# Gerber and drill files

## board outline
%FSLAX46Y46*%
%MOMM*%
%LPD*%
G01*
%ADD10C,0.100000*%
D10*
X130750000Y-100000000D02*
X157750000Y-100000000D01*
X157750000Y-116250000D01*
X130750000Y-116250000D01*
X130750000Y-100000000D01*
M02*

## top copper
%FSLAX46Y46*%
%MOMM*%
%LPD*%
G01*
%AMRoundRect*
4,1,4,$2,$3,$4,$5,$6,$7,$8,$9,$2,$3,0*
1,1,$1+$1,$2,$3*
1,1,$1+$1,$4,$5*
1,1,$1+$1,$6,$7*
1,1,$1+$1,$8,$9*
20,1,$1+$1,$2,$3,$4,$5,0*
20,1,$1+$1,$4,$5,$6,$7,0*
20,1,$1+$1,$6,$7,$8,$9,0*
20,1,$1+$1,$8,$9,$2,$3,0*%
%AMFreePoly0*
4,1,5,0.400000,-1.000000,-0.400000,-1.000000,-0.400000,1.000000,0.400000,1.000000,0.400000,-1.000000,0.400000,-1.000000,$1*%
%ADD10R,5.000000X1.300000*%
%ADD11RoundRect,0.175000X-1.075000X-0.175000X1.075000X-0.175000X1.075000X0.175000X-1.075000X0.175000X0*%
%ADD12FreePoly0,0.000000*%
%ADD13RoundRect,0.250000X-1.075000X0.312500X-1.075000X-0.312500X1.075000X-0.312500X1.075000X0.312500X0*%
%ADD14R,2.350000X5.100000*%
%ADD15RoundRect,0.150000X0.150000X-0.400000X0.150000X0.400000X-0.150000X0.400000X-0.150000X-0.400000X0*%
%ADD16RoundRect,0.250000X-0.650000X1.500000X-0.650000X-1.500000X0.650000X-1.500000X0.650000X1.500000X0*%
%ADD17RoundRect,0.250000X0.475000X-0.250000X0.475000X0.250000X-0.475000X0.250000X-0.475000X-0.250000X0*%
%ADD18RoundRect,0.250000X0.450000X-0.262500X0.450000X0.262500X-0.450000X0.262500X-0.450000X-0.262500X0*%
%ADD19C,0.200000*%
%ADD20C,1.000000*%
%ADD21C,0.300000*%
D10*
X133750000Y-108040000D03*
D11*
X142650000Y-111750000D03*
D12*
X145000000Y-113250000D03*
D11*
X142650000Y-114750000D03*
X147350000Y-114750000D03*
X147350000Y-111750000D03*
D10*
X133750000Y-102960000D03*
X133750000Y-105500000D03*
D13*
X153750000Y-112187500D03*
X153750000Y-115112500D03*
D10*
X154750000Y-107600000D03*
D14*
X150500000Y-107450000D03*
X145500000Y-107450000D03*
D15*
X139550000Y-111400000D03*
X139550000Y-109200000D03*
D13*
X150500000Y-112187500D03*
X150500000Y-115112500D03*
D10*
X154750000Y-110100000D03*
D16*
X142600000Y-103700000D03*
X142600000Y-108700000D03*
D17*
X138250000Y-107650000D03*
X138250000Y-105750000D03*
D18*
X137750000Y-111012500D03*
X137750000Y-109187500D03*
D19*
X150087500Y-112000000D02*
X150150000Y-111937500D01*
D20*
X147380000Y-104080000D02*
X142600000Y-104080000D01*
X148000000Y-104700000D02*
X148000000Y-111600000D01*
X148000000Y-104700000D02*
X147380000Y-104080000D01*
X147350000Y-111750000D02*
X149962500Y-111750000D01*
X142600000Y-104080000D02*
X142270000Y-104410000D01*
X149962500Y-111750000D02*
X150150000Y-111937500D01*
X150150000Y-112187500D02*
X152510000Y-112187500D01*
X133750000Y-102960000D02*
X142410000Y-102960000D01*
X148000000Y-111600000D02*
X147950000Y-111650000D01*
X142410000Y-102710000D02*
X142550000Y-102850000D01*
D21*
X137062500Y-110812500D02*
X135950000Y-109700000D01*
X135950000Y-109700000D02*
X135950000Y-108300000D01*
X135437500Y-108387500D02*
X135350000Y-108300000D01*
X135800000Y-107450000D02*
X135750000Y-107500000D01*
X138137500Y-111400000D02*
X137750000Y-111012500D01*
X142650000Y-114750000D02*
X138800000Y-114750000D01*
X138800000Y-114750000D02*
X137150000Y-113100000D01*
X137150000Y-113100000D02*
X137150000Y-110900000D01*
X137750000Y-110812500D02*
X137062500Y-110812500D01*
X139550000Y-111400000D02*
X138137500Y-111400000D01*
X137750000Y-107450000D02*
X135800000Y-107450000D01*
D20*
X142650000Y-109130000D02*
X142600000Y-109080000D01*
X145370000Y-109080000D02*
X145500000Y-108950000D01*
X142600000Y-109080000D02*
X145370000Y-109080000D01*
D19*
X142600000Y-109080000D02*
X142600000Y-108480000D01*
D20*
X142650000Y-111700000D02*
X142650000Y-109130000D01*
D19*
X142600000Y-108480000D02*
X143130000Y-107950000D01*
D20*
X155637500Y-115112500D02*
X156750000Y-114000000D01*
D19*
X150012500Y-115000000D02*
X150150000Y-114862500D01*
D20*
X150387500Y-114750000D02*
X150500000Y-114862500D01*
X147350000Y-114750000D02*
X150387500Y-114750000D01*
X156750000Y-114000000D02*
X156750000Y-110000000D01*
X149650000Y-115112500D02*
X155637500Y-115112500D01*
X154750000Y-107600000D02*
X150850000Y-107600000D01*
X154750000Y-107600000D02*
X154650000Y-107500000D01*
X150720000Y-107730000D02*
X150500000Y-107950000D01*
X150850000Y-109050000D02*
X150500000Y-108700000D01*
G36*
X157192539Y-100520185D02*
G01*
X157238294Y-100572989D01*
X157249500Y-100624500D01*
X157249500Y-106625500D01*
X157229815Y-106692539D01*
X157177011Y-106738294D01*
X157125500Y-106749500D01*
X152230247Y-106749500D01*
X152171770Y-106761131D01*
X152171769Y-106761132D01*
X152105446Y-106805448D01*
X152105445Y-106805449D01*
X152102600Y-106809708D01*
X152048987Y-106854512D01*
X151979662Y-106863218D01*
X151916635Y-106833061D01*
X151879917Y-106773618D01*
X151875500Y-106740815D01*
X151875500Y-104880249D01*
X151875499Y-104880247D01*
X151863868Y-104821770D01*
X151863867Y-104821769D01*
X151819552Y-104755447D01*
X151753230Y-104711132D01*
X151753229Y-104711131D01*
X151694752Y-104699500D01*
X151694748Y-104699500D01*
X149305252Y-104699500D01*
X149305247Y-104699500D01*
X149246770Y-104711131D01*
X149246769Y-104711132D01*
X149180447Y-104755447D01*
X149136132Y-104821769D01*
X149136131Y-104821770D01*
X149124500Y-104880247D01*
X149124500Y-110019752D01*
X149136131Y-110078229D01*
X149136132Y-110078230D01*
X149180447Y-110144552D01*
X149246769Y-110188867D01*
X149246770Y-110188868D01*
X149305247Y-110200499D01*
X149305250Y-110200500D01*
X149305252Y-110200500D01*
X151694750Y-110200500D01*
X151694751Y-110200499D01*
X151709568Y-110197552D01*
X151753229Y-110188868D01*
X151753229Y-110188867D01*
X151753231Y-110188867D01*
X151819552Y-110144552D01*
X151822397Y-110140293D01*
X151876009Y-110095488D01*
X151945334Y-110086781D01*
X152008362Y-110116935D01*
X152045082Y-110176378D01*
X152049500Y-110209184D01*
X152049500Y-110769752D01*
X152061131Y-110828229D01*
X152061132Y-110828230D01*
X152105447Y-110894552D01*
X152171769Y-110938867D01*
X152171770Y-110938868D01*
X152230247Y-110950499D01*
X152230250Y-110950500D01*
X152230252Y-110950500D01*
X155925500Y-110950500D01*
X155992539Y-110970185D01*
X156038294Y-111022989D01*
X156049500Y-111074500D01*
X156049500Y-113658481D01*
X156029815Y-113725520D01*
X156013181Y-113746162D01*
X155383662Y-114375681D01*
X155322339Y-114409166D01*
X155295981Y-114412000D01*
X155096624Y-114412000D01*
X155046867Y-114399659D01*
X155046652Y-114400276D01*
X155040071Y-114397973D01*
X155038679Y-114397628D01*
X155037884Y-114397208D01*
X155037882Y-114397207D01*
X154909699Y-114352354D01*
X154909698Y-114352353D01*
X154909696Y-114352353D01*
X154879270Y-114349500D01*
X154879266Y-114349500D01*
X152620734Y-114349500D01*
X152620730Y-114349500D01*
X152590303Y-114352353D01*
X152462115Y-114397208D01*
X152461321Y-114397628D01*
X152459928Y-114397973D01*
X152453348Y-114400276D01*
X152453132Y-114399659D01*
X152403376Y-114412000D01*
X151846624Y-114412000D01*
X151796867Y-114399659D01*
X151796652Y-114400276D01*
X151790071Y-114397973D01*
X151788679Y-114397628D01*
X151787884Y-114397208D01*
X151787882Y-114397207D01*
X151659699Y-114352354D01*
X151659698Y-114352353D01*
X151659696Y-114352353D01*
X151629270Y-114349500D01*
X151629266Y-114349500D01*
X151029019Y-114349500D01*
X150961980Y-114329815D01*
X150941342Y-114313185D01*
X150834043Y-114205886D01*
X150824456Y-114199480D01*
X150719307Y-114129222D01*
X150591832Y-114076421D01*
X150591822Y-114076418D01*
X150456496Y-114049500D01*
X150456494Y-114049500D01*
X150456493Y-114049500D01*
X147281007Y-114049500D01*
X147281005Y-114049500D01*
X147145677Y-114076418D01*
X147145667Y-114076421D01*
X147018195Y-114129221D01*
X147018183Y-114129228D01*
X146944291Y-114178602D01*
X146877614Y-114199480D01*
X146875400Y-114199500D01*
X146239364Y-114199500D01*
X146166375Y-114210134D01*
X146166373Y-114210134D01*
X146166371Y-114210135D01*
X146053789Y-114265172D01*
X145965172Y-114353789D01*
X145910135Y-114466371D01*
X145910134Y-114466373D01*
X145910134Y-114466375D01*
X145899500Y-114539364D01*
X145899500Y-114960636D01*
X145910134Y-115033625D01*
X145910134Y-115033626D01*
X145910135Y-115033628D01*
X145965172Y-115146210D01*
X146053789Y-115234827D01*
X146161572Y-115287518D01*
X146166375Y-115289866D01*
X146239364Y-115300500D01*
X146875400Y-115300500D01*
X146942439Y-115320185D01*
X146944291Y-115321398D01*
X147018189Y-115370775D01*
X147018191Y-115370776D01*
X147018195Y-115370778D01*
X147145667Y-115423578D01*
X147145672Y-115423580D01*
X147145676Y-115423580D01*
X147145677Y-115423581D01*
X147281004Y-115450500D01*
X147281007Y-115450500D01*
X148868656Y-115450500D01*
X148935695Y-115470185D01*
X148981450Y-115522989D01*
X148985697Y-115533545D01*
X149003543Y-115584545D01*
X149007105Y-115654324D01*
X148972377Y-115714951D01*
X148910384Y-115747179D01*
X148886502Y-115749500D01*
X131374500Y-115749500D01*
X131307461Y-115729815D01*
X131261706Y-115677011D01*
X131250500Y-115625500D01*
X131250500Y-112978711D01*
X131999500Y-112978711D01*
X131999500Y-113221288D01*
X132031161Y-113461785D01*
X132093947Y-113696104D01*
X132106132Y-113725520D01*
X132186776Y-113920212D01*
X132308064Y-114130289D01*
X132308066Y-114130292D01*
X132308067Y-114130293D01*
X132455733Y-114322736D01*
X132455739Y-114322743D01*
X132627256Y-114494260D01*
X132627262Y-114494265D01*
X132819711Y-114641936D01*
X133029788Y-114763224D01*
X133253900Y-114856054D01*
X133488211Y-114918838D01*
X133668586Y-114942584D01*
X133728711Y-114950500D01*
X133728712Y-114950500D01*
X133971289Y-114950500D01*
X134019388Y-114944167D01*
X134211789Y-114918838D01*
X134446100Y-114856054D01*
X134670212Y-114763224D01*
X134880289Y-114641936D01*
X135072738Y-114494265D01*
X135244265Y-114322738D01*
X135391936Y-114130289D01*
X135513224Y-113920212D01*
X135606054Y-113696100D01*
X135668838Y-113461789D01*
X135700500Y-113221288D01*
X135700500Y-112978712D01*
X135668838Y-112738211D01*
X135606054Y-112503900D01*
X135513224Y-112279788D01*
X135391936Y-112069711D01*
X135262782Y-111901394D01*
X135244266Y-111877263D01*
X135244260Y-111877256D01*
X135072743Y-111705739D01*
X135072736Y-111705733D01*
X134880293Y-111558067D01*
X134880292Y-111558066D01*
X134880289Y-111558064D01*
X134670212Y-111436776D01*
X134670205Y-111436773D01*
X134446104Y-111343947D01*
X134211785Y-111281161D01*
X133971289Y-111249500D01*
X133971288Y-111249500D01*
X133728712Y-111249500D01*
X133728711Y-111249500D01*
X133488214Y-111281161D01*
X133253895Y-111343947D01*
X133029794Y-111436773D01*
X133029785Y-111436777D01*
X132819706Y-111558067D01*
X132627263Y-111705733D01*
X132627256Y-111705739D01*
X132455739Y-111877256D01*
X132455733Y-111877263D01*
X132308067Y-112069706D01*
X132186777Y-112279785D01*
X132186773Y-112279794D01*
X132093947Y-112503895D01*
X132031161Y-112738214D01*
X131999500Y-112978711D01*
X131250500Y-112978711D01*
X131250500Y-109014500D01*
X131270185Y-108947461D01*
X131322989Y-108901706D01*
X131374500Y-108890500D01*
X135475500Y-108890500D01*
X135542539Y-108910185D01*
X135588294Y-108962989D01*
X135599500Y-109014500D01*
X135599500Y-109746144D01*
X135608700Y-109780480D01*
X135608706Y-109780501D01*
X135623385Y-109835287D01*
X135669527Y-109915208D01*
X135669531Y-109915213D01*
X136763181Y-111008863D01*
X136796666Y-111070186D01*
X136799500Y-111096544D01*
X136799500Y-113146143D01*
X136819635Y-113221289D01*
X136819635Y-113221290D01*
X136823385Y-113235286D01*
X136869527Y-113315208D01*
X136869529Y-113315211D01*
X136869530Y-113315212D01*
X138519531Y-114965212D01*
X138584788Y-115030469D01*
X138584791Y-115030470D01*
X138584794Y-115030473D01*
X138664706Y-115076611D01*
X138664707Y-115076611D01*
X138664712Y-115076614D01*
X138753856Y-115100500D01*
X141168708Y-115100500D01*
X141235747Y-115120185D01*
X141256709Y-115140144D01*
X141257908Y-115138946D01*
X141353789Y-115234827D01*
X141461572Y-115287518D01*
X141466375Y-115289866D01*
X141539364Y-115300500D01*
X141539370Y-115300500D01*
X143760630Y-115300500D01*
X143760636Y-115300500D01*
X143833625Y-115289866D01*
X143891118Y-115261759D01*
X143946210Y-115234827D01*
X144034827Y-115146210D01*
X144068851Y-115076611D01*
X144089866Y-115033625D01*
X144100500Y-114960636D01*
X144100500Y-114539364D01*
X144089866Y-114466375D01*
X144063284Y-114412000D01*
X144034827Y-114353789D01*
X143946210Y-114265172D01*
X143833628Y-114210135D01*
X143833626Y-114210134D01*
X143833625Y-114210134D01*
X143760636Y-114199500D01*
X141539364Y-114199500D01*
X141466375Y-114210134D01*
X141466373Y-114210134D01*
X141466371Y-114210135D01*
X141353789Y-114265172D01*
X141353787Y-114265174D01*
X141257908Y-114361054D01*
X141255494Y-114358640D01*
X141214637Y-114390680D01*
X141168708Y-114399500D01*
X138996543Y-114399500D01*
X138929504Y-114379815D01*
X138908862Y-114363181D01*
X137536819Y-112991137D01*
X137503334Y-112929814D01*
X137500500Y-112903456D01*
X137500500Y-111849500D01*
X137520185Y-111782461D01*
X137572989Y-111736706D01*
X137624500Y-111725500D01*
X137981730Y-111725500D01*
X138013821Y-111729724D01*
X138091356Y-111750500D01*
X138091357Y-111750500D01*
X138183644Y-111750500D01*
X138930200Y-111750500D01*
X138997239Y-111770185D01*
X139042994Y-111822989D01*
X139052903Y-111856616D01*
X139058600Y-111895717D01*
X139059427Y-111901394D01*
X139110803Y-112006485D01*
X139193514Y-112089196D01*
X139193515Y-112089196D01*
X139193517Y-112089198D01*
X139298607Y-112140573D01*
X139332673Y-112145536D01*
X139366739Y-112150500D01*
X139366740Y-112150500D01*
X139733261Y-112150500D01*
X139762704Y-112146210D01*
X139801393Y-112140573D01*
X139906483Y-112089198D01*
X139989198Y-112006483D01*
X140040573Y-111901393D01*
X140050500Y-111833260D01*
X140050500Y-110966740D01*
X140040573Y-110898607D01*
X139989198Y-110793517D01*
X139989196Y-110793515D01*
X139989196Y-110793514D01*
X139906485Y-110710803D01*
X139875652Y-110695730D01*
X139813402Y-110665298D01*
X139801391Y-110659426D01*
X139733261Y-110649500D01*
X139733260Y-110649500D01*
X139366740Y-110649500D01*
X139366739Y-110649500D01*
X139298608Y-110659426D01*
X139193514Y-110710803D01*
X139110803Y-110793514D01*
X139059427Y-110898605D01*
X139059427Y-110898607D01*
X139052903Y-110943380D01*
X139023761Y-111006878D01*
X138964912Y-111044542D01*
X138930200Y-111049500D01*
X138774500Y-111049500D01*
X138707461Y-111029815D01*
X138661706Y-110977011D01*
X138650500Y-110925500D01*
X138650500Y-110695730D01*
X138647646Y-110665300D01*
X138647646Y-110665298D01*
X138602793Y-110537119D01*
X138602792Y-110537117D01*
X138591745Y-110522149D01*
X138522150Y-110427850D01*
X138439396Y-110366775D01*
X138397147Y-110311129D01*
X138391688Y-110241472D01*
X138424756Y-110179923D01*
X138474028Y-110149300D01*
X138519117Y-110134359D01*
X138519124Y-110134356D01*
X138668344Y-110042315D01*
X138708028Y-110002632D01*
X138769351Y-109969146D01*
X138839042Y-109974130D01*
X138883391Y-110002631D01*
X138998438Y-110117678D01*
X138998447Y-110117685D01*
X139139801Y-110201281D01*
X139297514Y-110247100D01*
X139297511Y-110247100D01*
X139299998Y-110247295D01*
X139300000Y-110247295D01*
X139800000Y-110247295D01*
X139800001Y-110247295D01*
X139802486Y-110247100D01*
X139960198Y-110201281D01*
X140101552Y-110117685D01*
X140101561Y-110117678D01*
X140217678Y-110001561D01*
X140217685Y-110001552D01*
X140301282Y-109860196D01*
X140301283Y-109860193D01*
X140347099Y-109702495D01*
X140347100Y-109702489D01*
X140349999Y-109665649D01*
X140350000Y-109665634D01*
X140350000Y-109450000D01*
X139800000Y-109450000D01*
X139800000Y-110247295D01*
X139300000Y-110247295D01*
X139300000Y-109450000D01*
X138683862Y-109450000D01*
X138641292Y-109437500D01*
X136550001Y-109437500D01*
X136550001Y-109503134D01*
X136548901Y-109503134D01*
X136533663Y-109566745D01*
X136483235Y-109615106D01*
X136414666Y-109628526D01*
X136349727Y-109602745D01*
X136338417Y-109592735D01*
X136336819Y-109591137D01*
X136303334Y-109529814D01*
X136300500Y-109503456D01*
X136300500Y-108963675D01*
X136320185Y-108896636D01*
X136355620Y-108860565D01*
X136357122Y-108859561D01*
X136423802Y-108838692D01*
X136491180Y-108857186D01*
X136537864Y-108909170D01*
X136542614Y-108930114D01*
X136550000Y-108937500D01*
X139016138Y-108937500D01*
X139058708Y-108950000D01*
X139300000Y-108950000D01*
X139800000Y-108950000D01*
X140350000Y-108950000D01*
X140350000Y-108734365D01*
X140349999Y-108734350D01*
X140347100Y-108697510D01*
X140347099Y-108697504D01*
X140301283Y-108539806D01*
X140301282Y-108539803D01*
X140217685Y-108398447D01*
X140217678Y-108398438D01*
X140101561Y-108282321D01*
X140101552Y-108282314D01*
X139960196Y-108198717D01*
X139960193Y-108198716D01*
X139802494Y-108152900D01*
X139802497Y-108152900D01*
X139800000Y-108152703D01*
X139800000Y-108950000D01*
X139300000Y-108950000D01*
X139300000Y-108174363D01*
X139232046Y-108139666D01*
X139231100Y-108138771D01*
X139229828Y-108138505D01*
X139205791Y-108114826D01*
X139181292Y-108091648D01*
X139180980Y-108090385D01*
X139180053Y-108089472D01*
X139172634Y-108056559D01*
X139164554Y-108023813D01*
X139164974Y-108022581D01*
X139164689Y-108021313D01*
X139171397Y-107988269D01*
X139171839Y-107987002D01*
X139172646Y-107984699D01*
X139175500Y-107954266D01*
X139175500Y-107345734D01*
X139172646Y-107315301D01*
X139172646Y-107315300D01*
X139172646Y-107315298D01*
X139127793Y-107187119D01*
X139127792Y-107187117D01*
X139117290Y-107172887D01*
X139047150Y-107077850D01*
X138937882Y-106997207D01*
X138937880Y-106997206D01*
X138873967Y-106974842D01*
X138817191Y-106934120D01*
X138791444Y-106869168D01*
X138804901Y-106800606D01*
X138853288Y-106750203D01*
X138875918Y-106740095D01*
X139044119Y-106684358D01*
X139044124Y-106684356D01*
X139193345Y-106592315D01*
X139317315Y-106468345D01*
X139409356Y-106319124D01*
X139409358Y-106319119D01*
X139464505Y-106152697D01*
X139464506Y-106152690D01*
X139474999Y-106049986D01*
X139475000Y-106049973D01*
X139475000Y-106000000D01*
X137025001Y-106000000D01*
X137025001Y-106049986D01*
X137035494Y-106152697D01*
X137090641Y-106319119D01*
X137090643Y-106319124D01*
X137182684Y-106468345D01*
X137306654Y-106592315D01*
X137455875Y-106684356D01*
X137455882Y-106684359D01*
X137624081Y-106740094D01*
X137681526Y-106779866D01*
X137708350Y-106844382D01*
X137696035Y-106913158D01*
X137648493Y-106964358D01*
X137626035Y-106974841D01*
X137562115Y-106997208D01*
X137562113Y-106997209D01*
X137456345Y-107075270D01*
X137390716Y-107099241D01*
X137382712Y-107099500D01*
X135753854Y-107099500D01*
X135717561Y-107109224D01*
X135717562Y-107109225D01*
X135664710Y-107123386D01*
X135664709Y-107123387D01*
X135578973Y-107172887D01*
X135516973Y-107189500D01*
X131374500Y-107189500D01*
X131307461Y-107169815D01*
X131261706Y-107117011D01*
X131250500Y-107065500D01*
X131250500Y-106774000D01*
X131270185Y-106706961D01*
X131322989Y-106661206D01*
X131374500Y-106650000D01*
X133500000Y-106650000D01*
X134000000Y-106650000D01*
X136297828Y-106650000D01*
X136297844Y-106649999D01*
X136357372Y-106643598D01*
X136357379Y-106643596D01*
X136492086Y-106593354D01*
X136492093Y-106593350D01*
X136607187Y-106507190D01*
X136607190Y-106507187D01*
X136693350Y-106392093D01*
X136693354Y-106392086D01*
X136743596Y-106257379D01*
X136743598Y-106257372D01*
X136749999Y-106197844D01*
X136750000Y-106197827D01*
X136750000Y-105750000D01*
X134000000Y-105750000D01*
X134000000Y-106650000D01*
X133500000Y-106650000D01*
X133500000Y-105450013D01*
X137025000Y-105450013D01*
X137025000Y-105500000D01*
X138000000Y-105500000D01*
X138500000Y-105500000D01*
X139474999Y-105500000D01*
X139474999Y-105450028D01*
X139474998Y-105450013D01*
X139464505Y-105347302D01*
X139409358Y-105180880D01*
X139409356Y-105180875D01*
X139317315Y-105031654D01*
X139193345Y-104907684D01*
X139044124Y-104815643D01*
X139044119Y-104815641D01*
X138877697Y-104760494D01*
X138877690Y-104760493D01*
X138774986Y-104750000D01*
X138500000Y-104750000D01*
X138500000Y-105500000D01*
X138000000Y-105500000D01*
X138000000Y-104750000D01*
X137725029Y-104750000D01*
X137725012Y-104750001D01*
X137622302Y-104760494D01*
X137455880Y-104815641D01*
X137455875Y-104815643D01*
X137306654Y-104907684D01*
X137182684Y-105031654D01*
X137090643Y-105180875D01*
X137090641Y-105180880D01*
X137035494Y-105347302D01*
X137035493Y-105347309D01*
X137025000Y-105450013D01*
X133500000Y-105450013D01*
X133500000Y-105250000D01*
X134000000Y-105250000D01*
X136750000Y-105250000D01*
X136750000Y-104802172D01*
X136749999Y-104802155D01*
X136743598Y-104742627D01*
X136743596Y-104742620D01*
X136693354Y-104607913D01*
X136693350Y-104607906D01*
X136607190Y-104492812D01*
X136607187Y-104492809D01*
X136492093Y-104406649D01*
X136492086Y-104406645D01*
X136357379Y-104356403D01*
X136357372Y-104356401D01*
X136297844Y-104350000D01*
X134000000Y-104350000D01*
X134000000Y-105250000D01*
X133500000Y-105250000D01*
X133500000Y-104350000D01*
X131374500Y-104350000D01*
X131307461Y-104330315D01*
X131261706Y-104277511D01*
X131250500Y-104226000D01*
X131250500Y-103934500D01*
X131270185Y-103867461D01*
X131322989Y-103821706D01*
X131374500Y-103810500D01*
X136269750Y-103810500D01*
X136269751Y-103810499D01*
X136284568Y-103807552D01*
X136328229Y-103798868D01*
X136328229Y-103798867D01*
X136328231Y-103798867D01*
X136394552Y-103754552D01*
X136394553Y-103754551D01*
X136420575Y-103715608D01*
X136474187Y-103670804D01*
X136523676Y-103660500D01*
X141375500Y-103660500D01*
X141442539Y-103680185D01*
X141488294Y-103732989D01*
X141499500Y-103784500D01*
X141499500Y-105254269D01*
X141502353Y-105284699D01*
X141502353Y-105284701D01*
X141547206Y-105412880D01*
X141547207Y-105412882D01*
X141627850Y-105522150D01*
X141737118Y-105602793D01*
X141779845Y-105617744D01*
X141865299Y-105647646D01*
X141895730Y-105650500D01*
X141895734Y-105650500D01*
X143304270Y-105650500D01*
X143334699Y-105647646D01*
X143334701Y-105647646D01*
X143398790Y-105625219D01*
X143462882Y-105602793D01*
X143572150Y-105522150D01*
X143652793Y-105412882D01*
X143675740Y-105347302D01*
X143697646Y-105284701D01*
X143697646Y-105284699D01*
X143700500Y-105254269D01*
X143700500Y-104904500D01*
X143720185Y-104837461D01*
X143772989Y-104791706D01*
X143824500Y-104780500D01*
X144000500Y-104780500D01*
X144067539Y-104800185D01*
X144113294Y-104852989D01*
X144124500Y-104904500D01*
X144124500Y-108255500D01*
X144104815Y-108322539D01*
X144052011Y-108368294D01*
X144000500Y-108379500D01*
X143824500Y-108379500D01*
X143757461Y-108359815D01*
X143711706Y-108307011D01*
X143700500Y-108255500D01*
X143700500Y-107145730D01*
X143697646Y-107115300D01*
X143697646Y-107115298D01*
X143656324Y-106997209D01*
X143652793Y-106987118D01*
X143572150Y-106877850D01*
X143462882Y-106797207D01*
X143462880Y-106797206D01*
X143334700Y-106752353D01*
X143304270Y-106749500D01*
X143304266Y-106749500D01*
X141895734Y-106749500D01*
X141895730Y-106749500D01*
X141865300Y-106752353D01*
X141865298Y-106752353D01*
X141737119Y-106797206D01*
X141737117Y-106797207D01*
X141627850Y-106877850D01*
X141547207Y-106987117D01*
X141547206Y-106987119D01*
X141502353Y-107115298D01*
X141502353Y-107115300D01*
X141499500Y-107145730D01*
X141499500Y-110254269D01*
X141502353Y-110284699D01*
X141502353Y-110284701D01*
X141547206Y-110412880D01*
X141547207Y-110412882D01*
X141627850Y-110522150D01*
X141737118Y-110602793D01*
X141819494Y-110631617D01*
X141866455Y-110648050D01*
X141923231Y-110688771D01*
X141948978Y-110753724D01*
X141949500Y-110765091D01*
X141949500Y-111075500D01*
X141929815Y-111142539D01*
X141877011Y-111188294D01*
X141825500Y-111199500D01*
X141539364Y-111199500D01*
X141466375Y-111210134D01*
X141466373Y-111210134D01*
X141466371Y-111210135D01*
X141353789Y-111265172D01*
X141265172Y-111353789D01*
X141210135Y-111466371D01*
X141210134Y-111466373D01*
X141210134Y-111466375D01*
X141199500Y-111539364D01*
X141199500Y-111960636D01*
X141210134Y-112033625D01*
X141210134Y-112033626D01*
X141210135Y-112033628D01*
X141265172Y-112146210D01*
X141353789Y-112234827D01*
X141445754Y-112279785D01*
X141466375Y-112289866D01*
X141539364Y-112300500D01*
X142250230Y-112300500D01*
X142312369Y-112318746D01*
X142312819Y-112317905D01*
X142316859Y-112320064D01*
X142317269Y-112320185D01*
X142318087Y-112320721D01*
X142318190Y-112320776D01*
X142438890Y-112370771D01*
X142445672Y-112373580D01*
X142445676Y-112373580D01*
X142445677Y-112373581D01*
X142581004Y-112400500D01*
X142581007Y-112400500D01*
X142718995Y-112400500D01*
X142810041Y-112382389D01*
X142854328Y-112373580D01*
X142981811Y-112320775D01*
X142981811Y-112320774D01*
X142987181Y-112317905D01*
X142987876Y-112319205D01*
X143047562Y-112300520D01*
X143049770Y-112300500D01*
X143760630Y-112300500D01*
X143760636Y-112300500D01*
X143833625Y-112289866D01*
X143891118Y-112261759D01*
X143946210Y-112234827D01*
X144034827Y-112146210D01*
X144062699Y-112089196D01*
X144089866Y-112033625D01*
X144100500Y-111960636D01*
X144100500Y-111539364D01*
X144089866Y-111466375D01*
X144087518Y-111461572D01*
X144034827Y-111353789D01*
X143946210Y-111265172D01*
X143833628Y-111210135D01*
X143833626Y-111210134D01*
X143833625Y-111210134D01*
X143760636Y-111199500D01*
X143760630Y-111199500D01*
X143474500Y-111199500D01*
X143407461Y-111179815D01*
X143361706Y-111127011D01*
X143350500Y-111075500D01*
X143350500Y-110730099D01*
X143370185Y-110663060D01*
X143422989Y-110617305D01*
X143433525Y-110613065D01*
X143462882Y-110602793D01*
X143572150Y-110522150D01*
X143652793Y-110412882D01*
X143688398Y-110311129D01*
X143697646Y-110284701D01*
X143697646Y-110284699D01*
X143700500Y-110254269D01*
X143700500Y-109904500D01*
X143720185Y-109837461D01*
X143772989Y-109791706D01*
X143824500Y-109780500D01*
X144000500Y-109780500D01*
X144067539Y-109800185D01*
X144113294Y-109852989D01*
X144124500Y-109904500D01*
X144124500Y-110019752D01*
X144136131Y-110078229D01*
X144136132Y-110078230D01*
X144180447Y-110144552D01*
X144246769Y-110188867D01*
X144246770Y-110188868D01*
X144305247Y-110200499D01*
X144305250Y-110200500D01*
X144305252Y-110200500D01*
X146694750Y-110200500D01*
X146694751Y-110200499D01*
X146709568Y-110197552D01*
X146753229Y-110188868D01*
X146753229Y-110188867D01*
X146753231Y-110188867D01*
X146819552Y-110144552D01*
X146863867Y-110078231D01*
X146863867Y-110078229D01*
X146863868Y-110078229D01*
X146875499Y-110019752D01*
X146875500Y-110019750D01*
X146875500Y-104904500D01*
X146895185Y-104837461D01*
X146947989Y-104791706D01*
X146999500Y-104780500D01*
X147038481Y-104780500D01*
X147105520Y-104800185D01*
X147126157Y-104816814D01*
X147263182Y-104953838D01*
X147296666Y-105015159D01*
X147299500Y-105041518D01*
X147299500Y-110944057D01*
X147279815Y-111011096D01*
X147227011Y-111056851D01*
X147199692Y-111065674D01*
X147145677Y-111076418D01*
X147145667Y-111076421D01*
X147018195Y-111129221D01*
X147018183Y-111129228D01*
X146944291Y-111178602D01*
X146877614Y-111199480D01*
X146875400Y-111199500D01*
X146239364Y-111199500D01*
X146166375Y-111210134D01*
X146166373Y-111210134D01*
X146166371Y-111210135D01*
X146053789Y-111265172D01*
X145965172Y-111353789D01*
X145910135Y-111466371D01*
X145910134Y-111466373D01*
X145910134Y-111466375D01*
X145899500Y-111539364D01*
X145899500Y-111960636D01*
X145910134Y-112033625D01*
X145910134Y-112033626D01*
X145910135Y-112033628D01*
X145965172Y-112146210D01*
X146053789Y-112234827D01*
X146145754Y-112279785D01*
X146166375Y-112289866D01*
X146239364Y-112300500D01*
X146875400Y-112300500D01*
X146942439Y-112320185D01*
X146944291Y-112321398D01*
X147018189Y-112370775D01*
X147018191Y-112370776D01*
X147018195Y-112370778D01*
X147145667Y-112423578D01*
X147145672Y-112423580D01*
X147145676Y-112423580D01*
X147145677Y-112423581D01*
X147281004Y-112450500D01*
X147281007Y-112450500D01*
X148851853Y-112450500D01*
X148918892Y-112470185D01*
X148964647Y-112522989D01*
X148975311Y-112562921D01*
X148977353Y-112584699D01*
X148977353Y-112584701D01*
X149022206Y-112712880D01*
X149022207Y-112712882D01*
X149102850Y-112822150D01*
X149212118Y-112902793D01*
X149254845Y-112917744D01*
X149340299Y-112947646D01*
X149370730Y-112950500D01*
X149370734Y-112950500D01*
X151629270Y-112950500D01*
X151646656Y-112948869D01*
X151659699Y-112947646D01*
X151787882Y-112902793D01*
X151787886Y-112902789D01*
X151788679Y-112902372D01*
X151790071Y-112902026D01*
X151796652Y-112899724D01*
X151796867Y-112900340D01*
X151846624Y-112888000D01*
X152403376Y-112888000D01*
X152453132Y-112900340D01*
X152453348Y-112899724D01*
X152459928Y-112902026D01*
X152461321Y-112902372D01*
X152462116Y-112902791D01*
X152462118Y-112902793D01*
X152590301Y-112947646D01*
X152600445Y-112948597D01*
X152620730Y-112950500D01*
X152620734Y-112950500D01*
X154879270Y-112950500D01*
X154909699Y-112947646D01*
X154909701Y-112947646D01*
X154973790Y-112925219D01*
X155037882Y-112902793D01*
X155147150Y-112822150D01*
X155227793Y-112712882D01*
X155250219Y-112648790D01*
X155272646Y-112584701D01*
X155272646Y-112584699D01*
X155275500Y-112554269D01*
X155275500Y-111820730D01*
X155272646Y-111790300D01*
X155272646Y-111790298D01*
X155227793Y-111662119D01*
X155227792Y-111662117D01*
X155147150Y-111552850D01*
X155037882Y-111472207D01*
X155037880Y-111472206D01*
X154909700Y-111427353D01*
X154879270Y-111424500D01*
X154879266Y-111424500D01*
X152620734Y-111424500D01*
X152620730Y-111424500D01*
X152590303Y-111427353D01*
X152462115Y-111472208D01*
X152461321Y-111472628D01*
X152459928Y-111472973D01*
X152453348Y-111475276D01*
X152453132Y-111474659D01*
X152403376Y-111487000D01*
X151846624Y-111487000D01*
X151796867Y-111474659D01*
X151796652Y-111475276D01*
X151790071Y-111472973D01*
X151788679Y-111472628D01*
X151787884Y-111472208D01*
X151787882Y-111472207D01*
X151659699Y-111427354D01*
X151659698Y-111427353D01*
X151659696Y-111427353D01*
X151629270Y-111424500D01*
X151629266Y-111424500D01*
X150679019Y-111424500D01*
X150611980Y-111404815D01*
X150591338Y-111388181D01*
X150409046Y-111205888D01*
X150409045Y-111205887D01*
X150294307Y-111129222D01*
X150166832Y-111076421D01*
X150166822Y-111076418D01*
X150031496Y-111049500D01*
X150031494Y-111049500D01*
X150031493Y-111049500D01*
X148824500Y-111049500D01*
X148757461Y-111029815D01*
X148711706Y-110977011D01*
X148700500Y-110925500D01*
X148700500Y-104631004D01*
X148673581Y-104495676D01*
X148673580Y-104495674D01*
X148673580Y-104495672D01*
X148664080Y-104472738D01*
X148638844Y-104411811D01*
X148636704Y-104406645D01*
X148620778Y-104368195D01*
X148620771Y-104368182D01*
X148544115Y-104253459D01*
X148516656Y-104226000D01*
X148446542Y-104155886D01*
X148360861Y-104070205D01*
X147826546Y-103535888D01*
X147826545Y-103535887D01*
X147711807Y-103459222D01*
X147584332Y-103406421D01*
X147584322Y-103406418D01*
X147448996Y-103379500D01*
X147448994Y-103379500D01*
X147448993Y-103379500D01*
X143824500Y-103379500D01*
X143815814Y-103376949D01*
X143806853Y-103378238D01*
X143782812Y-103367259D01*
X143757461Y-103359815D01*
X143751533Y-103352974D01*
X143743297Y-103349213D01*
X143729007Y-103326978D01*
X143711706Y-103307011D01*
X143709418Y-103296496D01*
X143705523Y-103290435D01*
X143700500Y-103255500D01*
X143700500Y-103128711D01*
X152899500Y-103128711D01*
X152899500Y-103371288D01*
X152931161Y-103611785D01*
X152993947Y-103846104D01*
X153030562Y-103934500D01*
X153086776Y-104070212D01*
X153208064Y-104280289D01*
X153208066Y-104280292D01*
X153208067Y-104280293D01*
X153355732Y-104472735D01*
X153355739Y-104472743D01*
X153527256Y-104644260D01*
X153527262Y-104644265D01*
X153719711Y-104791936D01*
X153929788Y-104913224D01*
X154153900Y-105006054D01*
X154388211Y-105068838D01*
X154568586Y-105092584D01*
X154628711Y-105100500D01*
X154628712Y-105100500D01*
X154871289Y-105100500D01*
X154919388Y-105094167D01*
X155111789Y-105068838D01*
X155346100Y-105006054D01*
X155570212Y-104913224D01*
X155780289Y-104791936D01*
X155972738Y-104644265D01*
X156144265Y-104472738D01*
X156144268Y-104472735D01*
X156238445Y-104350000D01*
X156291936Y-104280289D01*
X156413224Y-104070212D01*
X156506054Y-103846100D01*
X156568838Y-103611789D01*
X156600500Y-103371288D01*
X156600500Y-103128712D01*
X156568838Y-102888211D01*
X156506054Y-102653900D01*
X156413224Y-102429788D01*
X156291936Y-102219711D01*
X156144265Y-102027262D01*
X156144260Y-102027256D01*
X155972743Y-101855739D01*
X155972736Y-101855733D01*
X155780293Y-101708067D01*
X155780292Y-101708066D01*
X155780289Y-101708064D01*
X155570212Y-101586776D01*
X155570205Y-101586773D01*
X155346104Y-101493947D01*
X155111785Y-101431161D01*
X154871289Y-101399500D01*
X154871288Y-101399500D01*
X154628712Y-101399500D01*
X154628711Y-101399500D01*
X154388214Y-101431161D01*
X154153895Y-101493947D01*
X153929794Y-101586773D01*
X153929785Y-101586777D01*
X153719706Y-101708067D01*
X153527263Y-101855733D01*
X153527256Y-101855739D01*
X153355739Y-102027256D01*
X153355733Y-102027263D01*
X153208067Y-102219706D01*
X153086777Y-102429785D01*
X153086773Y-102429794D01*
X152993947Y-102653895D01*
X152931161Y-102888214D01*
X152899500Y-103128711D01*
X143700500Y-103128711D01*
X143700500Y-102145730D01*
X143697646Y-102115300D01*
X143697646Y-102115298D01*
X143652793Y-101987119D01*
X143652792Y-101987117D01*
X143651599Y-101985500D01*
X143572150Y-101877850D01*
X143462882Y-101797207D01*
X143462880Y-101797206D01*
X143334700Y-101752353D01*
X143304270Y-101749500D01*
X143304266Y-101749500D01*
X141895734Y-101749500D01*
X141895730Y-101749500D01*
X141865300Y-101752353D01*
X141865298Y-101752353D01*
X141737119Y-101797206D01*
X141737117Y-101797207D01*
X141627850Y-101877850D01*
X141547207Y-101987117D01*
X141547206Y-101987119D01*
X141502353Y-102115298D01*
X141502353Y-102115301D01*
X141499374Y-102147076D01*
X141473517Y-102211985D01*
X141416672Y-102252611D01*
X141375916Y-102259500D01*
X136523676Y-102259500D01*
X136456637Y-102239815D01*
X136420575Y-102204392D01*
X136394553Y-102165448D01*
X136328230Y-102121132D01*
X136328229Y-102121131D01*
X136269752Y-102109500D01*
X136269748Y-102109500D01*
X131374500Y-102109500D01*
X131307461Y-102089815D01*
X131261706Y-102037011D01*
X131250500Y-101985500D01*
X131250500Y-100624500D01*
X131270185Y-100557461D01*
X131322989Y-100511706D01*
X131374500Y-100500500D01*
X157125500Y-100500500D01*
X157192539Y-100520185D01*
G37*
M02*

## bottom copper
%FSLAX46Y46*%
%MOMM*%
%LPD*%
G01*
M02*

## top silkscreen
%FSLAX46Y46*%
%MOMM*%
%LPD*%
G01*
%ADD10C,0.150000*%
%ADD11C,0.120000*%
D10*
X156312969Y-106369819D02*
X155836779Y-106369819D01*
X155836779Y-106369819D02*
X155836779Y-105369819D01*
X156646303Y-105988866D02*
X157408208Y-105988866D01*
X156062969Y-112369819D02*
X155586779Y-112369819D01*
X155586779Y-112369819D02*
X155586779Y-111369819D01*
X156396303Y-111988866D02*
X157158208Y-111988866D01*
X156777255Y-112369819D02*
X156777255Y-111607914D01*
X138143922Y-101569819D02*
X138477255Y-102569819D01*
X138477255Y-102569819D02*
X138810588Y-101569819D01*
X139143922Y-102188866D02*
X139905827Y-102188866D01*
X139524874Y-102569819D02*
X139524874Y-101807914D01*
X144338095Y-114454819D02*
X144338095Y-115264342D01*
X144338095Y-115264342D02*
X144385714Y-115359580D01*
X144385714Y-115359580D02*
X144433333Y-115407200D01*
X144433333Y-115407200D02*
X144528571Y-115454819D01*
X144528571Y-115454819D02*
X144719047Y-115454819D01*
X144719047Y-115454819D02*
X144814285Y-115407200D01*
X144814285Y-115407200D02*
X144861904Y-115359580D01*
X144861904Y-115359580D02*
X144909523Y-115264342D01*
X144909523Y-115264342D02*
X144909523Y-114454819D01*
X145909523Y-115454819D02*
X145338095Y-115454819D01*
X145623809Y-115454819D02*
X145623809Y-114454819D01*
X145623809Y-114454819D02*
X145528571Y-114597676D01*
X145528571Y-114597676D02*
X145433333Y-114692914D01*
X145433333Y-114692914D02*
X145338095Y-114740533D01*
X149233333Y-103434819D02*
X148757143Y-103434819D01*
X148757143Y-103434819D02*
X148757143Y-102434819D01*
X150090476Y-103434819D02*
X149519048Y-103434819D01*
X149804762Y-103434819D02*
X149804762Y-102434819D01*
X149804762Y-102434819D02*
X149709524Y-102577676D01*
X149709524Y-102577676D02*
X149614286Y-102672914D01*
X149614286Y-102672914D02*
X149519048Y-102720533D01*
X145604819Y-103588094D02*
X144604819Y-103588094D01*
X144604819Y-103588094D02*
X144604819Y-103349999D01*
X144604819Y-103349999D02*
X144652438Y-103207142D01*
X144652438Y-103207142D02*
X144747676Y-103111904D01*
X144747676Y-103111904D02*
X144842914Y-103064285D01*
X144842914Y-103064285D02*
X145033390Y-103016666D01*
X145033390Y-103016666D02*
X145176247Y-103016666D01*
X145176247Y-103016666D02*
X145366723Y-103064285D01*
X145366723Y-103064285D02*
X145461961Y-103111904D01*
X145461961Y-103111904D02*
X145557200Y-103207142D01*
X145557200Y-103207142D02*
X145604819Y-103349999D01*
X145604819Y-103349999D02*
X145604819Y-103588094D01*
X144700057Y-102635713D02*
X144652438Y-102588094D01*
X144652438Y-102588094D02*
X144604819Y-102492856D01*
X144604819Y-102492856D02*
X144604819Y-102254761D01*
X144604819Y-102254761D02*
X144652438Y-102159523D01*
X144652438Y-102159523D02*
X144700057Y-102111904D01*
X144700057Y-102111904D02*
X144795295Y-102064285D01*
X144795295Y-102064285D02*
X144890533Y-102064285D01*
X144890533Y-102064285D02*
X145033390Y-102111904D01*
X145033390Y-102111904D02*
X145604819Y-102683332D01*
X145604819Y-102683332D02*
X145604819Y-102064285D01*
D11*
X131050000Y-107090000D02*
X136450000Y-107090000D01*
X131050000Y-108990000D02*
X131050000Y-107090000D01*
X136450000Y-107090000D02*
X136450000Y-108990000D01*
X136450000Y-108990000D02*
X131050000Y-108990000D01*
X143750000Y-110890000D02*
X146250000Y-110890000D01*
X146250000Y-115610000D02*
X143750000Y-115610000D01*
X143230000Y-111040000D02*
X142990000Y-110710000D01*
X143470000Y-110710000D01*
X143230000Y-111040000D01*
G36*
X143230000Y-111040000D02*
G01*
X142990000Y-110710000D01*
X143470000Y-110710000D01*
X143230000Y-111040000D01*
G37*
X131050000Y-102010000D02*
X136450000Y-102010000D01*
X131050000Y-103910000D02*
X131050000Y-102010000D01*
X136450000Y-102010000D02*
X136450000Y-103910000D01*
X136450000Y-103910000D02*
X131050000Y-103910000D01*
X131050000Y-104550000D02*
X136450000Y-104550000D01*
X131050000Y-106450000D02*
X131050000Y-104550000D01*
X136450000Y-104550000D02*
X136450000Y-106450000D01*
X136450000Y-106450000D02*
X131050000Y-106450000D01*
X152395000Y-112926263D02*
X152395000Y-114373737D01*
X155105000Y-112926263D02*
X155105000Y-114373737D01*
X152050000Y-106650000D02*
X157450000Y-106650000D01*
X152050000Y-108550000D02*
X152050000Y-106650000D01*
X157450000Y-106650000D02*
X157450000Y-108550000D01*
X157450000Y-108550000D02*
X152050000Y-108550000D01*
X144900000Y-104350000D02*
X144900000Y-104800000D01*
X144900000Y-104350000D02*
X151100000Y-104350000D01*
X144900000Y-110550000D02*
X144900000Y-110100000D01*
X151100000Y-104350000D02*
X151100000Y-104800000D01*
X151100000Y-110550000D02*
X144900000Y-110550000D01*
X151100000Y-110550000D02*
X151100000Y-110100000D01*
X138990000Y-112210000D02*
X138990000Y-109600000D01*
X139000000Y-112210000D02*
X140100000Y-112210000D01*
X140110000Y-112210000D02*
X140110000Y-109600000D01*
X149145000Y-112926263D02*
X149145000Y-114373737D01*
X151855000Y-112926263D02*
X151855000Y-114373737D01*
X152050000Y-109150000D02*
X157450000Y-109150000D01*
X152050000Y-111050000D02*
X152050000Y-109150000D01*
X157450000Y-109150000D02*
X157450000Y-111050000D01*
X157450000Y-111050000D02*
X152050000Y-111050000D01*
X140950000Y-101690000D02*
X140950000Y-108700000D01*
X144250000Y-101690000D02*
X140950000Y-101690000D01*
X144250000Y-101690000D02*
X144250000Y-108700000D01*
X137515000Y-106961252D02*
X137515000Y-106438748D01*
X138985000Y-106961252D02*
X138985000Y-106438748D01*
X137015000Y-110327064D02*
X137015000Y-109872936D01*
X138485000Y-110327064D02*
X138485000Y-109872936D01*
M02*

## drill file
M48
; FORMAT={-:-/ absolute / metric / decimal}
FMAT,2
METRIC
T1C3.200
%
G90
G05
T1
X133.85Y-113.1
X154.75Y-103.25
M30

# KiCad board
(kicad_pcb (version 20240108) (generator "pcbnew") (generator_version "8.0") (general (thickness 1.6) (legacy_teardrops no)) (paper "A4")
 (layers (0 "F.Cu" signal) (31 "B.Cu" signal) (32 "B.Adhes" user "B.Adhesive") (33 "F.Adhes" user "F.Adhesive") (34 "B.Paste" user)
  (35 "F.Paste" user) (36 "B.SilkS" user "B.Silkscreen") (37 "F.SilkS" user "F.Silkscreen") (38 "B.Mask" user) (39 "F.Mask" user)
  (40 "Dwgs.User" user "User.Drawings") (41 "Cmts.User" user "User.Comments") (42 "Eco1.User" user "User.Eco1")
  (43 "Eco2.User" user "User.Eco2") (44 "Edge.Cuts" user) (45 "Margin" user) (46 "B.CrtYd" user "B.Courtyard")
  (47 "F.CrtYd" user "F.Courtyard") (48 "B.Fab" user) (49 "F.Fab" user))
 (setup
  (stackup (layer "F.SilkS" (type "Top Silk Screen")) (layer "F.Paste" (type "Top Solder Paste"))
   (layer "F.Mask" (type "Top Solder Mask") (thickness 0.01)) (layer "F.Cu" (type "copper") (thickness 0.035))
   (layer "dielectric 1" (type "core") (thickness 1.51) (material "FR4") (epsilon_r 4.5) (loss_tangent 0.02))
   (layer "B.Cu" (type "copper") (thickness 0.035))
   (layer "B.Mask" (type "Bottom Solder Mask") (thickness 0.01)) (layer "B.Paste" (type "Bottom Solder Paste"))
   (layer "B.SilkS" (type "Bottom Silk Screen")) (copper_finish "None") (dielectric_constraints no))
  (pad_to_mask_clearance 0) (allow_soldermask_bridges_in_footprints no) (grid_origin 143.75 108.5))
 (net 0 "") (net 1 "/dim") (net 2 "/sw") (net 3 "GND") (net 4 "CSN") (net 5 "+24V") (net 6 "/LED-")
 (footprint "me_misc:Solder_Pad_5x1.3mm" (layer "F.Cu") (at 133.75 108.04)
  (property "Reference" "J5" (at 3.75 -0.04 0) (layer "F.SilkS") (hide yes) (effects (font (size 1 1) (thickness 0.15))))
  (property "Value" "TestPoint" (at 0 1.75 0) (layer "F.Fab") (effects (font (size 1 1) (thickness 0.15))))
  (fp_line (start -2.7 -0.95) (end 2.7 -0.95) (stroke (width 0.12) (type solid)) (layer "F.SilkS"))
  (fp_line (start -2.7 0.95) (end -2.7 -0.95) (stroke (width 0.12) (type solid)) (layer "F.SilkS"))
  (fp_line (start 2.7 -0.95) (end 2.7 0.95) (stroke (width 0.12) (type solid)) (layer "F.SilkS"))
  (fp_line (start 2.7 0.95) (end -2.7 0.95) (stroke (width 0.12) (type solid)) (layer "F.SilkS"))
  (pad "1" smd rect (at 0 0) (size 5 1.3) (layers "F.Cu" "F.Mask") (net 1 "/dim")))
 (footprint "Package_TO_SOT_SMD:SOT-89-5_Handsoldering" (layer "F.Cu") (at 145 113.25)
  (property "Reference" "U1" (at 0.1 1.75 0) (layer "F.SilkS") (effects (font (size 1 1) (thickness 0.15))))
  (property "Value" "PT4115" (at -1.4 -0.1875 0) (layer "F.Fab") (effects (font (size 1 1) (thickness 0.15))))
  (fp_line (start -1.25 -2.36) (end 1.25 -2.36) (stroke (width 0.12) (type solid)) (layer "F.SilkS"))
  (fp_line (start 1.25 2.36) (end -1.25 2.36) (stroke (width 0.12) (type solid)) (layer "F.SilkS"))
  (fp_poly
   (pts (xy -1.77 -2.21) (xy -2.01 -2.54) (xy -1.53 -2.54) (xy -1.77 -2.21)) (stroke (width 0.12) (type solid)) (fill solid)
   (layer "F.SilkS"))
  (pad "1" smd roundrect (at -2.35 -1.5) (size 2.5 0.7) (layers "F.Cu" "F.Paste" "F.Mask") (roundrect_rratio 0.25) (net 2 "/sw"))
  (pad "2" smd custom (at 0 0) (size 0.8 2) (layers "F.Cu" "F.Paste" "F.Mask") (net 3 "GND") (zone_connect 2) (thermal_bridge_angle 45)
   (options (clearance outline) (anchor rect)) (primitives))
  (pad "3" smd roundrect (at -2.35 1.5) (size 2.5 0.7) (layers "F.Cu" "F.Paste" "F.Mask") (roundrect_rratio 0.25) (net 1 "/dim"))
  (pad "4" smd roundrect (at 2.35 1.5) (size 2.5 0.7) (layers "F.Cu" "F.Paste" "F.Mask") (roundrect_rratio 0.25) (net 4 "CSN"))
  (pad "5" smd roundrect (at 2.35 -1.5) (size 2.5 0.7) (layers "F.Cu" "F.Paste" "F.Mask") (roundrect_rratio 0.25) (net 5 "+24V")))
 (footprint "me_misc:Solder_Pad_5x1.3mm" (layer "F.Cu") (at 133.75 102.96)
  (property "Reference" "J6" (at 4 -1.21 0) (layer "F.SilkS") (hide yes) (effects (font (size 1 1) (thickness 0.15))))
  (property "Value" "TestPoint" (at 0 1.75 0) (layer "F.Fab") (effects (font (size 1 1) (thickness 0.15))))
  (fp_line (start -2.7 -0.95) (end 2.7 -0.95) (stroke (width 0.12) (type solid)) (layer "F.SilkS"))
  (fp_line (start -2.7 0.95) (end -2.7 -0.95) (stroke (width 0.12) (type solid)) (layer "F.SilkS"))
  (fp_line (start 2.7 -0.95) (end 2.7 0.95) (stroke (width 0.12) (type solid)) (layer "F.SilkS"))
  (fp_line (start 2.7 0.95) (end -2.7 0.95) (stroke (width 0.12) (type solid)) (layer "F.SilkS"))
  (pad "1" smd rect (at 0 0) (size 5 1.3) (layers "F.Cu" "F.Mask") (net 5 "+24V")))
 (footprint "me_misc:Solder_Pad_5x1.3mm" (layer "F.Cu") (at 133.75 105.5)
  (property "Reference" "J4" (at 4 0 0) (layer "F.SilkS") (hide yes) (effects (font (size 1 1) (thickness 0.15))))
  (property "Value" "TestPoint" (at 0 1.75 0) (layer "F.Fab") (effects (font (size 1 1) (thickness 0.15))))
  (fp_line (start -2.7 -0.95) (end 2.7 -0.95) (stroke (width 0.12) (type solid)) (layer "F.SilkS"))
  (fp_line (start -2.7 0.95) (end -2.7 -0.95) (stroke (width 0.12) (type solid)) (layer "F.SilkS"))
  (fp_line (start 2.7 -0.95) (end 2.7 0.95) (stroke (width 0.12) (type solid)) (layer "F.SilkS"))
  (fp_line (start 2.7 0.95) (end -2.7 0.95) (stroke (width 0.12) (type solid)) (layer "F.SilkS"))
  (pad "1" smd rect (at 0 0) (size 5 1.3) (layers "F.Cu" "F.Mask") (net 3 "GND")))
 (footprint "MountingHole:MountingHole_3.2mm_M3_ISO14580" (layer "F.Cu") (at 154.75 103.25)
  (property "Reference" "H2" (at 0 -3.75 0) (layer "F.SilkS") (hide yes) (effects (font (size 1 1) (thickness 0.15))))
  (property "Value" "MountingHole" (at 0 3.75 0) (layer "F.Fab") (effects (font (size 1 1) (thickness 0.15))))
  (pad "" np_thru_hole circle (at 0 0) (size 3.2 3.2) (drill 3.2) (layers "*.Cu" "*.Mask")))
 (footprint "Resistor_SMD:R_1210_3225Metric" (layer "F.Cu") (at 153.75 113.65 -90)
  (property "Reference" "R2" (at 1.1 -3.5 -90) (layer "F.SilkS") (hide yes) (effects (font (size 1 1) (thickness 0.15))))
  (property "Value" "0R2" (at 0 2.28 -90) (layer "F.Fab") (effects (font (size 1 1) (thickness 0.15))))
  (fp_line (start -0.723737 1.355) (end 0.723737 1.355) (stroke (width 0.12) (type solid)) (layer "F.SilkS"))
  (fp_line (start -0.723737 -1.355) (end 0.723737 -1.355) (stroke (width 0.12) (type solid)) (layer "F.SilkS"))
  (pad "1" smd roundrect (at -1.4625 0 270) (size 1.125 2.65) (layers "F.Cu" "F.Paste" "F.Mask") (roundrect_rratio 0.222222) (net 5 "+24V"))
  (pad "2" smd roundrect (at 1.4625 0 270) (size 1.125 2.65) (layers "F.Cu" "F.Paste" "F.Mask") (roundrect_rratio 0.222222) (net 4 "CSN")))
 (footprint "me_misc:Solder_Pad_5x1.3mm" (layer "F.Cu") (at 154.75 107.6 180)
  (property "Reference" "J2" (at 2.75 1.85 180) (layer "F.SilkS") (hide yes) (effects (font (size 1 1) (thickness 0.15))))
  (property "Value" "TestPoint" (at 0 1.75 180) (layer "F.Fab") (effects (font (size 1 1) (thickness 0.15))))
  (fp_line (start 2.7 0.95) (end -2.7 0.95) (stroke (width 0.12) (type solid)) (layer "F.SilkS"))
  (fp_line (start 2.7 -0.95) (end 2.7 0.95) (stroke (width 0.12) (type solid)) (layer "F.SilkS"))
  (fp_line (start -2.7 0.95) (end -2.7 -0.95) (stroke (width 0.12) (type solid)) (layer "F.SilkS"))
  (fp_line (start -2.7 -0.95) (end 2.7 -0.95) (stroke (width 0.12) (type solid)) (layer "F.SilkS"))
  (pad "1" smd rect (at 0 0 180) (size 5 1.3) (layers "F.Cu" "F.Mask") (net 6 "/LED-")))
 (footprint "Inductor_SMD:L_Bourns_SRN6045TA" (layer "F.Cu") (at 148 107.45 180)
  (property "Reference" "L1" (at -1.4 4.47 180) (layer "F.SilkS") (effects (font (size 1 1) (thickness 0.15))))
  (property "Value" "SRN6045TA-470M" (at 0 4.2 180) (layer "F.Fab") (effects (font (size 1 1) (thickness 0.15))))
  (fp_line (start 3.1 3.1) (end 3.1 2.65) (stroke (width 0.12) (type solid)) (layer "F.SilkS"))
  (fp_line (start 3.1 3.1) (end -3.1 3.1) (stroke (width 0.12) (type solid)) (layer "F.SilkS"))
  (fp_line (start 3.1 -3.1) (end 3.1 -2.65) (stroke (width 0.12) (type solid)) (layer "F.SilkS"))
  (fp_line (start -3.1 3.1) (end -3.1 2.65) (stroke (width 0.12) (type solid)) (layer "F.SilkS"))
  (fp_line (start -3.1 -3.1) (end 3.1 -3.1) (stroke (width 0.12) (type solid)) (layer "F.SilkS"))
  (fp_line (start -3.1 -3.1) (end -3.1 -2.65) (stroke (width 0.12) (type solid)) (layer "F.SilkS"))
  (pad "1" smd rect (at -2.5 0 180) (size 2.35 5.1) (layers "F.Cu" "F.Paste" "F.Mask") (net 6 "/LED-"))
  (pad "2" smd rect (at 2.5 0 180) (size 2.35 5.1) (layers "F.Cu" "F.Paste" "F.Mask") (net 2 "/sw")))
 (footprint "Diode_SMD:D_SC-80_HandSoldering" (layer "F.Cu") (at 139.55 110.3 90)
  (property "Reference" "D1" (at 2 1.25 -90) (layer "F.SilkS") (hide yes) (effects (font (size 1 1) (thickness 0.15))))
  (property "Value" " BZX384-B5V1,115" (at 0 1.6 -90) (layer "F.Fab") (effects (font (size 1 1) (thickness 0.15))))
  (fp_line (start -1.91 -0.56) (end 0.7 -0.56) (stroke (width 0.12) (type solid)) (layer "F.SilkS"))
  (fp_line (start -1.91 -0.55) (end -1.91 0.55) (stroke (width 0.12) (type solid)) (layer "F.SilkS"))
  (fp_line (start -1.91 0.56) (end 0.7 0.56) (stroke (width 0.12) (type solid)) (layer "F.SilkS"))
  (pad "1" smd roundrect (at -1.1 0 90) (size 1.1 0.6) (layers "F.Cu" "F.Paste" "F.Mask") (roundrect_rratio 0.25) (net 1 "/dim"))
  (pad "2" smd roundrect (at 1.1 0 90) (size 1.1 0.6) (layers "F.Cu" "F.Paste" "F.Mask") (roundrect_rratio 0.25) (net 3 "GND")))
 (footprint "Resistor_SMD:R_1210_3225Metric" (layer "F.Cu") (at 150.5 113.65 -90)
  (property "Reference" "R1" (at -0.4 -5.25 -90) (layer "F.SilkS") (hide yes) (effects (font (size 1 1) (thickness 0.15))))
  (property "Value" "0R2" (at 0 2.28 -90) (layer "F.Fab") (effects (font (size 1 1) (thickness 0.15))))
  (fp_line (start -0.723737 1.355) (end 0.723737 1.355) (stroke (width 0.12) (type solid)) (layer "F.SilkS"))
  (fp_line (start -0.723737 -1.355) (end 0.723737 -1.355) (stroke (width 0.12) (type solid)) (layer "F.SilkS"))
  (pad "1" smd roundrect (at -1.4625 0 270) (size 1.125 2.65) (layers "F.Cu" "F.Paste" "F.Mask") (roundrect_rratio 0.222222) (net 5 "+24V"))
  (pad "2" smd roundrect (at 1.4625 0 270) (size 1.125 2.65) (layers "F.Cu" "F.Paste" "F.Mask") (roundrect_rratio 0.222222) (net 4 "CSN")))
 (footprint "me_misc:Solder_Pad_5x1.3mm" (layer "F.Cu") (at 154.75 110.1 180)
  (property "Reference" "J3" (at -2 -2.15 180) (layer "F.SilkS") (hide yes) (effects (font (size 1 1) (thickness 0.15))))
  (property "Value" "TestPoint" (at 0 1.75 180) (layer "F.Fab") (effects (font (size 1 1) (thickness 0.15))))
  (fp_line (start 2.7 0.95) (end -2.7 0.95) (stroke (width 0.12) (type solid)) (layer "F.SilkS"))
  (fp_line (start 2.7 -0.95) (end 2.7 0.95) (stroke (width 0.12) (type solid)) (layer "F.SilkS"))
  (fp_line (start -2.7 0.95) (end -2.7 -0.95) (stroke (width 0.12) (type solid)) (layer "F.SilkS"))
  (fp_line (start -2.7 -0.95) (end 2.7 -0.95) (stroke (width 0.12) (type solid)) (layer "F.SilkS"))
  (pad "1" smd rect (at 0 0 180) (size 5 1.3) (layers "F.Cu" "F.Mask") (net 4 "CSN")))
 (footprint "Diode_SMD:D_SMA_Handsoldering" (layer "F.Cu") (at 142.6 106.2 -90)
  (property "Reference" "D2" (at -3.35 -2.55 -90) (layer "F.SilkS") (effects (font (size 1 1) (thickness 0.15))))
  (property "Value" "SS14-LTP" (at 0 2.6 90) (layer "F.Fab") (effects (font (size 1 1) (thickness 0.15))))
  (fp_line (start -4.51 1.65) (end 2.5 1.65) (stroke (width 0.12) (type solid)) (layer "F.SilkS"))
  (fp_line (start -4.51 -1.65) (end -4.51 1.65) (stroke (width 0.12) (type solid)) (layer "F.SilkS"))
  (fp_line (start -4.51 -1.65) (end 2.5 -1.65) (stroke (width 0.12) (type solid)) (layer "F.SilkS"))
  (pad "1" smd roundrect (at -2.5 0 270) (size 3.5 1.8) (layers "F.Cu" "F.Paste" "F.Mask") (roundrect_rratio 0.1388888889) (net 5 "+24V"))
  (pad "2" smd roundrect (at 2.5 0 270) (size 3.5 1.8) (layers "F.Cu" "F.Paste" "F.Mask") (roundrect_rratio 0.1388888889) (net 2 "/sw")))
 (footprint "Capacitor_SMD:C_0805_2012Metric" (layer "F.Cu") (at 138.25 106.7 90)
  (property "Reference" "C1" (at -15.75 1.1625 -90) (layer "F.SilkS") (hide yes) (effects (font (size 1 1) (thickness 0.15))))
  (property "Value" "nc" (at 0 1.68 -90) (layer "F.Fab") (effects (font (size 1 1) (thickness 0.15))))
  (fp_line (start -0.261252 -0.735) (end 0.261252 -0.735) (stroke (width 0.12) (type solid)) (layer "F.SilkS"))
  (fp_line (start -0.261252 0.735) (end 0.261252 0.735) (stroke (width 0.12) (type solid)) (layer "F.SilkS"))
  (pad "1" smd roundrect (at -0.95 0 90) (size 1 1.45) (layers "F.Cu" "F.Paste" "F.Mask") (roundrect_rratio 0.25) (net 1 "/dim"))
  (pad "2" smd roundrect (at 0.95 0 90) (size 1 1.45) (layers "F.Cu" "F.Paste" "F.Mask") (roundrect_rratio 0.25) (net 3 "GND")))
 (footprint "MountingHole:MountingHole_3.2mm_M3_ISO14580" (layer "F.Cu") (at 133.85 113.1)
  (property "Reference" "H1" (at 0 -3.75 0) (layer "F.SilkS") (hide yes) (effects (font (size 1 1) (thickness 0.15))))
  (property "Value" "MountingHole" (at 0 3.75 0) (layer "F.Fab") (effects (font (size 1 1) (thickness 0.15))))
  (pad "" np_thru_hole circle (at 0 0) (size 3.2 3.2) (drill 3.2) (layers "*.Cu" "*.Mask")))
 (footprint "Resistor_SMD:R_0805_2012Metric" (layer "F.Cu") (at 137.75 110.1 90)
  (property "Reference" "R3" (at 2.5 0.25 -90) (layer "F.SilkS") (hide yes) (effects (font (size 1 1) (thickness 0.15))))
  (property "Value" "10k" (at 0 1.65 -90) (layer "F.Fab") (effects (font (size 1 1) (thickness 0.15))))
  (fp_line (start -0.227064 -0.735) (end 0.227064 -0.735) (stroke (width 0.12) (type solid)) (layer "F.SilkS"))
  (fp_line (start -0.227064 0.735) (end 0.227064 0.735) (stroke (width 0.12) (type solid)) (layer "F.SilkS"))
  (pad "1" smd roundrect (at -0.9125 0 90) (size 1.025 1.4) (layers "F.Cu" "F.Paste" "F.Mask") (roundrect_rratio 0.243902) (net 1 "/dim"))
  (pad "2" smd roundrect (at 0.9125 0 90) (size 1.025 1.4) (layers "F.Cu" "F.Paste" "F.Mask") (roundrect_rratio 0.243902) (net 3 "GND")))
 (gr_rect (start 130.75 100) (end 157.75 116.25) (stroke (width 0.1) (type default)) (fill none) (layer "Edge.Cuts"))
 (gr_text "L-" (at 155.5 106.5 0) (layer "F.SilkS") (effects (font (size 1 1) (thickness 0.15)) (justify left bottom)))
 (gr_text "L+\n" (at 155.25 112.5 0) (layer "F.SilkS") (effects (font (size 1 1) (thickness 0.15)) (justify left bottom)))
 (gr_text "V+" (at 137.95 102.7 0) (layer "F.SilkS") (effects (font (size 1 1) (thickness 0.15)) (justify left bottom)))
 (segment (start 150.0875 112) (end 150.15 111.9375) (width 0.2) (layer "F.Cu") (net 5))
 (segment (start 147.38 104.08) (end 142.6 104.08) (width 1) (layer "F.Cu") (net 5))
 (segment (start 148 104.7) (end 148 111.6) (width 1) (layer "F.Cu") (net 5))
 (segment (start 148 104.7) (end 147.38 104.08) (width 1) (layer "F.Cu") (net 5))
 (segment (start 147.35 111.75) (end 149.9625 111.75) (width 1) (layer "F.Cu") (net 5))
 (segment (start 142.6 104.08) (end 142.27 104.41) (width 1) (layer "F.Cu") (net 5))
 (segment (start 149.9625 111.75) (end 150.15 111.9375) (width 1) (layer "F.Cu") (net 5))
 (segment (start 150.15 112.1875) (end 152.51 112.1875) (width 1) (layer "F.Cu") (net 5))
 (segment (start 133.75 102.96) (end 142.41 102.96) (width 1) (layer "F.Cu") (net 5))
 (segment (start 148 111.6) (end 147.95 111.65) (width 1) (layer "F.Cu") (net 5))
 (segment (start 142.41 102.71) (end 142.55 102.85) (width 1) (layer "F.Cu") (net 5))
 (segment (start 137.0625 110.8125) (end 135.95 109.7) (width 0.3) (layer "F.Cu") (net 1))
 (segment (start 135.95 109.7) (end 135.95 108.3) (width 0.3) (layer "F.Cu") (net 1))
 (segment (start 135.4375 108.3875) (end 135.35 108.3) (width 0.3) (layer "F.Cu") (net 1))
 (segment (start 135.8 107.45) (end 135.75 107.5) (width 0.3) (layer "F.Cu") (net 1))
 (segment (start 138.1375 111.4) (end 137.75 111.0125) (width 0.3) (layer "F.Cu") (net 1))
 (segment (start 142.65 114.75) (end 138.8 114.75) (width 0.3) (layer "F.Cu") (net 1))
 (segment (start 138.8 114.75) (end 137.15 113.1) (width 0.3) (layer "F.Cu") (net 1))
 (segment (start 137.15 113.1) (end 137.15 110.9) (width 0.3) (layer "F.Cu") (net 1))
 (segment (start 137.75 110.8125) (end 137.0625 110.8125) (width 0.3) (layer "F.Cu") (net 1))
 (segment (start 139.55 111.4) (end 138.1375 111.4) (width 0.3) (layer "F.Cu") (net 1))
 (segment (start 137.75 107.45) (end 135.8 107.45) (width 0.3) (layer "F.Cu") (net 1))
 (segment (start 142.65 109.13) (end 142.6 109.08) (width 1) (layer "F.Cu") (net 2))
 (segment (start 145.37 109.08) (end 145.5 108.95) (width 1) (layer "F.Cu") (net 2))
 (segment (start 142.6 109.08) (end 145.37 109.08) (width 1) (layer "F.Cu") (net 2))
 (segment (start 142.6 109.08) (end 142.6 108.48) (width 0.2) (layer "F.Cu") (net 2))
 (segment (start 142.65 111.7) (end 142.65 109.13) (width 1) (layer "F.Cu") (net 2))
 (segment (start 142.6 108.48) (end 143.13 107.95) (width 0.2) (layer "F.Cu") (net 2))
 (segment (start 155.6375 115.1125) (end 156.75 114) (width 1) (layer "F.Cu") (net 4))
 (segment (start 150.0125 115) (end 150.15 114.8625) (width 0.2) (layer "F.Cu") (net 4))
 (segment (start 150.3875 114.75) (end 150.5 114.8625) (width 1) (layer "F.Cu") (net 4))
 (segment (start 147.35 114.75) (end 150.3875 114.75) (width 1) (layer "F.Cu") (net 4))
 (segment (start 156.75 114) (end 156.75 110) (width 1) (layer "F.Cu") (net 4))
 (segment (start 149.65 115.1125) (end 155.6375 115.1125) (width 1) (layer "F.Cu") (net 4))
 (segment (start 154.75 107.6) (end 150.85 107.6) (width 1) (layer "F.Cu") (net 6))
 (segment (start 154.75 107.6) (end 154.65 107.5) (width 1) (layer "F.Cu") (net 6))
 (segment (start 150.72 107.73) (end 150.5 107.95) (width 1) (layer "F.Cu") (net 6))
 (segment (start 150.85 109.05) (end 150.5 108.7) (width 1) (layer "F.Cu") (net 6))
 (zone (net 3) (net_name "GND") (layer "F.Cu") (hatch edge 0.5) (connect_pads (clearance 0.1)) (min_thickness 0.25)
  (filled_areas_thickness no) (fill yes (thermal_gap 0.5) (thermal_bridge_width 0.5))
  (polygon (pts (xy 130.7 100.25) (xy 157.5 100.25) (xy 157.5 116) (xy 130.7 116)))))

